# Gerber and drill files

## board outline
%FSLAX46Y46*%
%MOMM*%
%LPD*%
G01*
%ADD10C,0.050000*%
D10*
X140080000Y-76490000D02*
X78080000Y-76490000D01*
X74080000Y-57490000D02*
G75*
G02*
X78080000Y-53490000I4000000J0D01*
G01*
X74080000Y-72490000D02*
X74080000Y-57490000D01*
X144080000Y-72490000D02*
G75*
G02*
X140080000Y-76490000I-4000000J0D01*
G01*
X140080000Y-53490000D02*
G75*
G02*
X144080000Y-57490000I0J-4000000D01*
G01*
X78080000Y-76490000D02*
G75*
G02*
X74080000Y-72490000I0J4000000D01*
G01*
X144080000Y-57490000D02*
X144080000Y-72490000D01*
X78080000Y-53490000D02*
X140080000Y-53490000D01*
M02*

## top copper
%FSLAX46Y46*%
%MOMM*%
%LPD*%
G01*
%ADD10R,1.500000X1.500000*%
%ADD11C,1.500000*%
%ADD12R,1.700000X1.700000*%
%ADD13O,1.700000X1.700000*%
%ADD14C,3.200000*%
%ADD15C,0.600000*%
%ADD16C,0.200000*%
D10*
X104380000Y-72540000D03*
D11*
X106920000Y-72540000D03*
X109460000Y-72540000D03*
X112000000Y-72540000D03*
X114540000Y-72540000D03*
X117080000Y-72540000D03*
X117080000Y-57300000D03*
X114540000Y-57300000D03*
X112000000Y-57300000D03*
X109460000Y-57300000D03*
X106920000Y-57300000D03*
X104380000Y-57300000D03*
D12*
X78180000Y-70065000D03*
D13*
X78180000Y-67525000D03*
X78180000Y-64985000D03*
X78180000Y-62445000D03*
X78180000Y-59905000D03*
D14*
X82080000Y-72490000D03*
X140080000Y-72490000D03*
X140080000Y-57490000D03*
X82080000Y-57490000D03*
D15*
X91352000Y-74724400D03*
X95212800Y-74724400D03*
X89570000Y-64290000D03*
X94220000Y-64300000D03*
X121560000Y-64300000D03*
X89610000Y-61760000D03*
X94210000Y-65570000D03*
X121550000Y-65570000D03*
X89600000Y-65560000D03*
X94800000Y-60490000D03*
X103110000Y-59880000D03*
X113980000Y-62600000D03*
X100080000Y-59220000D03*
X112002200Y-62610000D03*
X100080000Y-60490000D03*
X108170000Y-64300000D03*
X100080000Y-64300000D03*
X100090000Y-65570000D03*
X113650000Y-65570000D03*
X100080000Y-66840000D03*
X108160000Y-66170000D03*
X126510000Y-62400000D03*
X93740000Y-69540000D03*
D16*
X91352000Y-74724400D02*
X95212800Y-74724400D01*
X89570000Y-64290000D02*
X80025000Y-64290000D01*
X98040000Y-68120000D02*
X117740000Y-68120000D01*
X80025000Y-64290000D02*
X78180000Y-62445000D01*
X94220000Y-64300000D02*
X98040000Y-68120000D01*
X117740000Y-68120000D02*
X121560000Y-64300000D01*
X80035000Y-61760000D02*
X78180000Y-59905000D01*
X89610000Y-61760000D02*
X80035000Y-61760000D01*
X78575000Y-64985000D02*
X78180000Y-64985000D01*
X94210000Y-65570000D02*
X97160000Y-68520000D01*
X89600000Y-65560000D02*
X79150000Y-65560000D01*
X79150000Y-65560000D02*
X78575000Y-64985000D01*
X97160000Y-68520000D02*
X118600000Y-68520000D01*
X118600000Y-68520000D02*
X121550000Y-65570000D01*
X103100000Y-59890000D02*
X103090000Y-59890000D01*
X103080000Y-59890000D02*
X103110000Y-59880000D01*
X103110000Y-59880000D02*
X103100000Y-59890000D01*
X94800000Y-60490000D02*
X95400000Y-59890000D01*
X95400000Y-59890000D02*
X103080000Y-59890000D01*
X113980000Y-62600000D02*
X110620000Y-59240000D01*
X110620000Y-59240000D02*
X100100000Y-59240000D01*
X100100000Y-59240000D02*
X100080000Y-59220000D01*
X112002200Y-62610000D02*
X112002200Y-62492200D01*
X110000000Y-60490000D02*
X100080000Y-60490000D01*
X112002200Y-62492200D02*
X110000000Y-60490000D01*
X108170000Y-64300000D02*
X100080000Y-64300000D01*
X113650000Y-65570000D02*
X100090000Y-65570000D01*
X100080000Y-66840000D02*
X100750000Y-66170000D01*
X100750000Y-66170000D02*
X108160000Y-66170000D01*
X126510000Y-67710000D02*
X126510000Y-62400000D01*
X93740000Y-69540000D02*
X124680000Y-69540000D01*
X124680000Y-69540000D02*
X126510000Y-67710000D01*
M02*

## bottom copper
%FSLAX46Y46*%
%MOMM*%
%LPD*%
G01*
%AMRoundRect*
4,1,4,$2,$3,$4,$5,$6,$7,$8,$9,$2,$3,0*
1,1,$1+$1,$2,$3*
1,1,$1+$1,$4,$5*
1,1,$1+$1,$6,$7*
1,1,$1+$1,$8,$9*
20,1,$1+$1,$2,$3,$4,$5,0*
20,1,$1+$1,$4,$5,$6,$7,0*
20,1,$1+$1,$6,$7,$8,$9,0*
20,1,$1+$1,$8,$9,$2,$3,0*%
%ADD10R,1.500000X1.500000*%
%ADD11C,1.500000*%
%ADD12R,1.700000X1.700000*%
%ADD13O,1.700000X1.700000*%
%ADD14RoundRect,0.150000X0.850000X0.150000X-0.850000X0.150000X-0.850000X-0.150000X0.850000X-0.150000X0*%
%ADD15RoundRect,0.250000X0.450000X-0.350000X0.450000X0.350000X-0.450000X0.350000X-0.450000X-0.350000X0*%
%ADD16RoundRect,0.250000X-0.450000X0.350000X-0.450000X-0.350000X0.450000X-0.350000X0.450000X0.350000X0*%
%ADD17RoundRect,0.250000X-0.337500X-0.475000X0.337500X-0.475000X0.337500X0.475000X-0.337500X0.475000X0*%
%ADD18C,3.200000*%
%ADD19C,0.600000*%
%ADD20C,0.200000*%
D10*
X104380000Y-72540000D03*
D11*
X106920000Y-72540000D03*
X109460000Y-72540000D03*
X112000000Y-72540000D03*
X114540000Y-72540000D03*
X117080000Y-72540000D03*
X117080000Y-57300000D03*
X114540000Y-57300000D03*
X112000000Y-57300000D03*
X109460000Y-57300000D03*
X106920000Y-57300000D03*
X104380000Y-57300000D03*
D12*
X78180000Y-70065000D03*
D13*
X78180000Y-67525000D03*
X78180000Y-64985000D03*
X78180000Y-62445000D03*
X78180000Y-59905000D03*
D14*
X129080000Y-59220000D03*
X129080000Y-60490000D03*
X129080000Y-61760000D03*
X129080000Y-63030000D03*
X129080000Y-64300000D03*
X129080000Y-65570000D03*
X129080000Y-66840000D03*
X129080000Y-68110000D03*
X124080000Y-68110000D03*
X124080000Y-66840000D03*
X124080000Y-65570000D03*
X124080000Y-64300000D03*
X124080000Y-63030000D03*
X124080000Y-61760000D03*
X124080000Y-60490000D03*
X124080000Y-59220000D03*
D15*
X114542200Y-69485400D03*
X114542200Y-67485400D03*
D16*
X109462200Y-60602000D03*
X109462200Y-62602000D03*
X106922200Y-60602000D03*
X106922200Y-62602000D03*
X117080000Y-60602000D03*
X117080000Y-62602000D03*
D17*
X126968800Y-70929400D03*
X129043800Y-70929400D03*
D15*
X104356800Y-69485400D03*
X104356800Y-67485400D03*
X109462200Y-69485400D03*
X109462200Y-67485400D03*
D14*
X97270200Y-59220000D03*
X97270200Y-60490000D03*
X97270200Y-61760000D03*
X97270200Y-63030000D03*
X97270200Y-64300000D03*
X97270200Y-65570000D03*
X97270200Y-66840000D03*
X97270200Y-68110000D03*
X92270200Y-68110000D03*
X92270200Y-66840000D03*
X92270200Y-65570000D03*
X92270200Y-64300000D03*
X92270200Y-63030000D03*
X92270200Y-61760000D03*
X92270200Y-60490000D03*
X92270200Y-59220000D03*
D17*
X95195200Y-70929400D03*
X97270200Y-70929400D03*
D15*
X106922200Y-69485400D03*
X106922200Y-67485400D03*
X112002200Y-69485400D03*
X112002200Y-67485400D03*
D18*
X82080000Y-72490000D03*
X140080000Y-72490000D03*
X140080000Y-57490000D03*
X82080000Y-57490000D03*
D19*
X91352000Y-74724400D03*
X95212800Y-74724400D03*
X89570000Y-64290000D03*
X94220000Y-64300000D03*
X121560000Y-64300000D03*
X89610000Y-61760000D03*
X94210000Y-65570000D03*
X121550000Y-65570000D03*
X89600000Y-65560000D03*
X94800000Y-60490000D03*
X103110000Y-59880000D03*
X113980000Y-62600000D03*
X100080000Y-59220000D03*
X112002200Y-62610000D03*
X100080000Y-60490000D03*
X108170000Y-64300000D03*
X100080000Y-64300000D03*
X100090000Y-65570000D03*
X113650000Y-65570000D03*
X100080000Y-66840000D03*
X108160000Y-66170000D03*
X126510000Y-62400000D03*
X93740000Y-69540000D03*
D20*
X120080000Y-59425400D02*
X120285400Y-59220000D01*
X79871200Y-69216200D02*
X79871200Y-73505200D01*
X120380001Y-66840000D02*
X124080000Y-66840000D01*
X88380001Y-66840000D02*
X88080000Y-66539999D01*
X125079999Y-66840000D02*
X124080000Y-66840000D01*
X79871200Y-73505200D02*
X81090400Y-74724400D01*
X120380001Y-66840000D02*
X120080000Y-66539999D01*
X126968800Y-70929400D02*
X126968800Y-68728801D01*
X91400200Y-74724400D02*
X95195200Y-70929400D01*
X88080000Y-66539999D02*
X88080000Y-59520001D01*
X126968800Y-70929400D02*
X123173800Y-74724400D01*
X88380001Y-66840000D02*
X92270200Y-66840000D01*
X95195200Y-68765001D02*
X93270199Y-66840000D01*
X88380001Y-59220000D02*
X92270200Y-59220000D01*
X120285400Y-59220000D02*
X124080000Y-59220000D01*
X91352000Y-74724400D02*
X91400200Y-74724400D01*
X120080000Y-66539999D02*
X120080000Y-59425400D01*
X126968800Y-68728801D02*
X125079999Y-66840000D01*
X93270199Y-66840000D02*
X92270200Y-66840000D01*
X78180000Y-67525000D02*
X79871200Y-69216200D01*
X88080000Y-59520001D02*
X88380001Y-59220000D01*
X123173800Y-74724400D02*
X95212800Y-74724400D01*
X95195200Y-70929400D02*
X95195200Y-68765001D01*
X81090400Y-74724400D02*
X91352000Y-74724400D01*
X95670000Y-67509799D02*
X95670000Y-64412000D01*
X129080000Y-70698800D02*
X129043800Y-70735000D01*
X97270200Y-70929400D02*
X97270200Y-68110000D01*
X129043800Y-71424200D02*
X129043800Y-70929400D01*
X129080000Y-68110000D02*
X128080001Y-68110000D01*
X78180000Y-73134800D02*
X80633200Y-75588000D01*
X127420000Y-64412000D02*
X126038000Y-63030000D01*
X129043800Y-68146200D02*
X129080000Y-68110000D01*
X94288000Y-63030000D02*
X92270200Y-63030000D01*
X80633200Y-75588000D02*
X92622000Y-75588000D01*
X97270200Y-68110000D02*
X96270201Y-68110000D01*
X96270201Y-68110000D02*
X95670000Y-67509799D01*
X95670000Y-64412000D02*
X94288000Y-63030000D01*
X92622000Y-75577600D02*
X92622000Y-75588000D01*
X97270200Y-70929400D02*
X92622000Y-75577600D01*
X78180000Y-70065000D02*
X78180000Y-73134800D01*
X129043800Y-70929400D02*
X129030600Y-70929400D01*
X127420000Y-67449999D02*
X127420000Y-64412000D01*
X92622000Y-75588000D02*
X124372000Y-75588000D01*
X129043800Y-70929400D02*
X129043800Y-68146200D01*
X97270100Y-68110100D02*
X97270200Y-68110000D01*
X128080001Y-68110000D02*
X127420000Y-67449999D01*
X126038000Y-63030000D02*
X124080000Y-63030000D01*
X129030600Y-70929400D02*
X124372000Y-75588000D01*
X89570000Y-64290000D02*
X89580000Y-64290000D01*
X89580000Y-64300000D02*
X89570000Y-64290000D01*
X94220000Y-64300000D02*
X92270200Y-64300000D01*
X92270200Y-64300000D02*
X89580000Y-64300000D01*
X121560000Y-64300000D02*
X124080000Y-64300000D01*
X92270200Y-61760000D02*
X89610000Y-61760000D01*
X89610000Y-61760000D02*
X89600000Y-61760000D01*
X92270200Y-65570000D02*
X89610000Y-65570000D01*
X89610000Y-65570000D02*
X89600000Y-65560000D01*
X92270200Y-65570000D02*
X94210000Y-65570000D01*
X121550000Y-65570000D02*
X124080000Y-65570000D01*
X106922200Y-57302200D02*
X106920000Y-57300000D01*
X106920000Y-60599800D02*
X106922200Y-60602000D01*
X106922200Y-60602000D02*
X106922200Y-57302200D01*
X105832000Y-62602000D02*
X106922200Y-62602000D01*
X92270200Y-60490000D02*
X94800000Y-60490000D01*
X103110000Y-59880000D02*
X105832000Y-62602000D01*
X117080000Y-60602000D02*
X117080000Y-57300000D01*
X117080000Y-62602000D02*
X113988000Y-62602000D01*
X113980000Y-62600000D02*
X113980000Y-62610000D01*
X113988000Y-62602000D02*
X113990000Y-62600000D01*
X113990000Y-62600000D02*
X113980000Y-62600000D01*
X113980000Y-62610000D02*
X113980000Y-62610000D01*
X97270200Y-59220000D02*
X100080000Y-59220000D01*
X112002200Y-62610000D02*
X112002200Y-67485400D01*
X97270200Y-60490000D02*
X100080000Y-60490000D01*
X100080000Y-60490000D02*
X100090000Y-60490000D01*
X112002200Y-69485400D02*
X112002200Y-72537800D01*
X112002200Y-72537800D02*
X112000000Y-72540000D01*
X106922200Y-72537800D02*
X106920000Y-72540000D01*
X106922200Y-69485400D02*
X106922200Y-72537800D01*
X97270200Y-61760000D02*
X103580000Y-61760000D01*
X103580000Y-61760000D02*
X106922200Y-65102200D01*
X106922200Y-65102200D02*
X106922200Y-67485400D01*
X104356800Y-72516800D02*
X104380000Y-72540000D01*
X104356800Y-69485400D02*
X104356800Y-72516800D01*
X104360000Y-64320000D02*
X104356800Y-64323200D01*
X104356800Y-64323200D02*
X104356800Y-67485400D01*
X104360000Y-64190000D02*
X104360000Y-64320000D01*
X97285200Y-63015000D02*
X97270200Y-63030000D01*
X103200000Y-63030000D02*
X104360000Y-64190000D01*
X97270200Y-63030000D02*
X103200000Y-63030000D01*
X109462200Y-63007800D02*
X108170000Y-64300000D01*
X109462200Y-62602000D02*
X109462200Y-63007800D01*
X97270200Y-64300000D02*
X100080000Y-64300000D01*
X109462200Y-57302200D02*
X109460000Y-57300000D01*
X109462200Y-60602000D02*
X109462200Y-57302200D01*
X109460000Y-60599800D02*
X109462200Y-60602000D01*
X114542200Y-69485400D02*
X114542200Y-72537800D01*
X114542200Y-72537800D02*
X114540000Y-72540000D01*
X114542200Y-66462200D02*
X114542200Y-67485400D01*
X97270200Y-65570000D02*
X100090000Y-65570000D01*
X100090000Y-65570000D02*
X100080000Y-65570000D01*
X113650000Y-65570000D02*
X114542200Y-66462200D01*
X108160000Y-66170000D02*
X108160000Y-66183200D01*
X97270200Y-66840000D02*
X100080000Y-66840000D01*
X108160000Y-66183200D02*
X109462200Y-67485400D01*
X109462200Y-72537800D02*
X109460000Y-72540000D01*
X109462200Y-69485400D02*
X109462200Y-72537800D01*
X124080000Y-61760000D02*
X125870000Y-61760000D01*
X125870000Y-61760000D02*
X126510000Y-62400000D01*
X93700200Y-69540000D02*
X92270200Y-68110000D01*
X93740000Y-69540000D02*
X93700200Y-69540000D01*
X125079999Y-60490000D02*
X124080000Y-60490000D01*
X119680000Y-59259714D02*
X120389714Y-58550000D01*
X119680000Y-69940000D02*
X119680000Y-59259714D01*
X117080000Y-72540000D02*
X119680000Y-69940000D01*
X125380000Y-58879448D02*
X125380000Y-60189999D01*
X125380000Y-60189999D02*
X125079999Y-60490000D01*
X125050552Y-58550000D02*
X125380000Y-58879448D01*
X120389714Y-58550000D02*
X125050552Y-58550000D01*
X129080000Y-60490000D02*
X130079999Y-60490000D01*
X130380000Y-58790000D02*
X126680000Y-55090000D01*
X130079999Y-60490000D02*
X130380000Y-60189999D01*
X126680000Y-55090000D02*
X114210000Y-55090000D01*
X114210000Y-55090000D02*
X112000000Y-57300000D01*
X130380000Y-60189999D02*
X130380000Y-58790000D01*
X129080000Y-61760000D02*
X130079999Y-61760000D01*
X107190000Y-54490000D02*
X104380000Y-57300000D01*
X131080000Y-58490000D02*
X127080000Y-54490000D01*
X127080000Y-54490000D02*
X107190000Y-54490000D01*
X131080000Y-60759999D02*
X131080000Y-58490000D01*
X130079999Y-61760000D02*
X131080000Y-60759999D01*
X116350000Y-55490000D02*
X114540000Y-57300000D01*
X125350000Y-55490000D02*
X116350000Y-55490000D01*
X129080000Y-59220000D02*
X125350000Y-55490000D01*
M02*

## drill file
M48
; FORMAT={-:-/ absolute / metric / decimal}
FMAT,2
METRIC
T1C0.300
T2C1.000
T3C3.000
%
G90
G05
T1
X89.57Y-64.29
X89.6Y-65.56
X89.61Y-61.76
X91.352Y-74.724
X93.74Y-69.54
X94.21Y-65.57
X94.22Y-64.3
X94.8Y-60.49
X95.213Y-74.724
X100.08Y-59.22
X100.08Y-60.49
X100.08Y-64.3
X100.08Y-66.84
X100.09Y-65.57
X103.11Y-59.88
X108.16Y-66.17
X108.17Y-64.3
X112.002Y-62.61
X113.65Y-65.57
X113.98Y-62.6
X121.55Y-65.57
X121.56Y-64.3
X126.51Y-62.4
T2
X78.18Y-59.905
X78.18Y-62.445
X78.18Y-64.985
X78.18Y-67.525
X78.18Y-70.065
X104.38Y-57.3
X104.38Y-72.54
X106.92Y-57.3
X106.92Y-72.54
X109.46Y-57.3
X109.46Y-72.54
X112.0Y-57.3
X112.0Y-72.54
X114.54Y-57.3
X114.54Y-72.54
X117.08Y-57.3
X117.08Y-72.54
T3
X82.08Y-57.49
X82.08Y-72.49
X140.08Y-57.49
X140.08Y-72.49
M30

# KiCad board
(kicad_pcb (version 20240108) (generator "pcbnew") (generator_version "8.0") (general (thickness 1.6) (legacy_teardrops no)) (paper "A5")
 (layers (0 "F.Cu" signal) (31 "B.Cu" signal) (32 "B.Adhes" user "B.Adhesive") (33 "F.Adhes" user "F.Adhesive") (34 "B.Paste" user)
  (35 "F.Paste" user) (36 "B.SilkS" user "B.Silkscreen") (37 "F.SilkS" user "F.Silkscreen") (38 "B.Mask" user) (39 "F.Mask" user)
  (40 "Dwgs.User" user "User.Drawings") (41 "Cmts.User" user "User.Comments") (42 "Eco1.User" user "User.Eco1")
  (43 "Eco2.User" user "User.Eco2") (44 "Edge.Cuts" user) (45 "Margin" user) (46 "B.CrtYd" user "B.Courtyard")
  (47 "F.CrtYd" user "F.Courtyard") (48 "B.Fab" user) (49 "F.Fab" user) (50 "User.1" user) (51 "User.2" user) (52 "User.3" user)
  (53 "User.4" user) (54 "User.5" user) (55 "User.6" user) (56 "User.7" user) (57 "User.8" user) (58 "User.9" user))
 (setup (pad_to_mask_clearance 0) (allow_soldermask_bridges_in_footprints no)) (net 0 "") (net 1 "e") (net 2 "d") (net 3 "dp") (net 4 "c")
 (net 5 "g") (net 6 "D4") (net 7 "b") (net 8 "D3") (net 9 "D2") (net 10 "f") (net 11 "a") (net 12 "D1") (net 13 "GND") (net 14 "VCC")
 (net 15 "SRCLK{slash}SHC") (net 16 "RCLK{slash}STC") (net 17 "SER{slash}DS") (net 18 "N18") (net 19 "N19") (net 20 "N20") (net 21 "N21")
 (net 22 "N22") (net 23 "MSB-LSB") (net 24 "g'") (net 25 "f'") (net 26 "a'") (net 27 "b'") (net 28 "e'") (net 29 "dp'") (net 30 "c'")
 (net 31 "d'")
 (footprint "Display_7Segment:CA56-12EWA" (layer "F.Cu") (at 104.38 72.54 90)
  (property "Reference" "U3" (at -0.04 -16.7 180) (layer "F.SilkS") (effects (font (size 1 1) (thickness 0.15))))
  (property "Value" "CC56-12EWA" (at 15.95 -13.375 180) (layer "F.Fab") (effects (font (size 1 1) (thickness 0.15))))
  (pad "1" thru_hole rect (at 0 0 90) (size 1.5 1.5) (drill 1) (layers "*.Cu" "*.Mask") (remove_unused_layers no) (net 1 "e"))
  (pad "2" thru_hole circle (at 0 2.54 90) (size 1.5 1.5) (drill 1) (layers "*.Cu" "*.Mask") (remove_unused_layers no) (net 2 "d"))
  (pad "3" thru_hole circle (at 0 5.08 90) (size 1.5 1.5) (drill 1) (layers "*.Cu" "*.Mask") (remove_unused_layers no) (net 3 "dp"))
  (pad "4" thru_hole circle (at 0 7.62 90) (size 1.5 1.5) (drill 1) (layers "*.Cu" "*.Mask") (remove_unused_layers no) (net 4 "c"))
  (pad "5" thru_hole circle (at 0 10.16 90) (size 1.5 1.5) (drill 1) (layers "*.Cu" "*.Mask") (remove_unused_layers no) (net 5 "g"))
  (pad "6" thru_hole circle (at 0 12.7 90) (size 1.5 1.5) (drill 1) (layers "*.Cu" "*.Mask") (remove_unused_layers no) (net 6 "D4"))
  (pad "7" thru_hole circle (at 15.24 12.7 90) (size 1.5 1.5) (drill 1) (layers "*.Cu" "*.Mask") (remove_unused_layers no) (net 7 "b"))
  (pad "8" thru_hole circle (at 15.24 10.16 90) (size 1.5 1.5) (drill 1) (layers "*.Cu" "*.Mask") (remove_unused_layers no) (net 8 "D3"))
  (pad "9" thru_hole circle (at 15.24 7.62 90) (size 1.5 1.5) (drill 1) (layers "*.Cu" "*.Mask") (remove_unused_layers no) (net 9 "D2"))
  (pad "10" thru_hole circle (at 15.24 5.08 90) (size 1.5 1.5) (drill 1) (layers "*.Cu" "*.Mask") (remove_unused_layers no) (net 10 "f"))
  (pad "11" thru_hole circle (at 15.24 2.54 90) (size 1.5 1.5) (drill 1) (layers "*.Cu" "*.Mask") (remove_unused_layers no) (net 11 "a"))
  (pad "12" thru_hole circle (at 15.24 0 90) (size 1.5 1.5) (drill 1) (layers "*.Cu" "*.Mask") (remove_unused_layers no) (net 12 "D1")))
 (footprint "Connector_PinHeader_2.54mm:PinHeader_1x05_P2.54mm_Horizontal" (layer "F.Cu") (at 78.18 70.065 180)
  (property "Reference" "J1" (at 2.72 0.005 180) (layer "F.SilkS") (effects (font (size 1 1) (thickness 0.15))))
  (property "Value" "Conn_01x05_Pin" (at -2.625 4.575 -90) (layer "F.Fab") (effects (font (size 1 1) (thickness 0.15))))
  (pad "1" thru_hole rect (at 0 0 180) (size 1.7 1.7) (drill 1) (layers "*.Cu" "*.Mask") (remove_unused_layers no) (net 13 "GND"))
  (pad "2" thru_hole oval (at 0 2.54 180) (size 1.7 1.7) (drill 1) (layers "*.Cu" "*.Mask") (remove_unused_layers no) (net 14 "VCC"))
  (pad "3" thru_hole oval (at 0 5.08 180) (size 1.7 1.7) (drill 1) (layers "*.Cu" "*.Mask") (remove_unused_layers no)
   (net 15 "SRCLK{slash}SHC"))
  (pad "4" thru_hole oval (at 0 7.62 180) (size 1.7 1.7) (drill 1) (layers "*.Cu" "*.Mask") (remove_unused_layers no)
   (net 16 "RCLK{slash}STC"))
  (pad "5" thru_hole oval (at 0 10.16 180) (size 1.7 1.7) (drill 1) (layers "*.Cu" "*.Mask") (remove_unused_layers no)
   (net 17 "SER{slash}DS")))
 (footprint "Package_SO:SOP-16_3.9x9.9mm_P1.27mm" (layer "B.Cu") (at 126.58 63.665 180)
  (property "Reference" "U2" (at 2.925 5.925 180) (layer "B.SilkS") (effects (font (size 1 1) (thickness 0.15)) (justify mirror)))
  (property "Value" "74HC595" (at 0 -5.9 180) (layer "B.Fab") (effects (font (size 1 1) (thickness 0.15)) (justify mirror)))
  (pad "1" smd roundrect (at -2.5 4.445 180) (size 2 0.6) (layers "B.Cu" "B.Paste" "B.Mask") (roundrect_rratio 0.25) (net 8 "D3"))
  (pad "2" smd roundrect (at -2.5 3.175 180) (size 2 0.6) (layers "B.Cu" "B.Paste" "B.Mask") (roundrect_rratio 0.25) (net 9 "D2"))
  (pad "3" smd roundrect (at -2.5 1.905 180) (size 2 0.6) (layers "B.Cu" "B.Paste" "B.Mask") (roundrect_rratio 0.25) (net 12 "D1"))
  (pad "4" smd roundrect (at -2.5 0.635 180) (size 2 0.6) (layers "B.Cu" "B.Paste" "B.Mask") (roundrect_rratio 0.25) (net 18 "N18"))
  (pad "5" smd roundrect (at -2.5 -0.635 180) (size 2 0.6) (layers "B.Cu" "B.Paste" "B.Mask") (roundrect_rratio 0.25) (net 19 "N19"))
  (pad "6" smd roundrect (at -2.5 -1.905 180) (size 2 0.6) (layers "B.Cu" "B.Paste" "B.Mask") (roundrect_rratio 0.25) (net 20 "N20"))
  (pad "7" smd roundrect (at -2.5 -3.175 180) (size 2 0.6) (layers "B.Cu" "B.Paste" "B.Mask") (roundrect_rratio 0.25) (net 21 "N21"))
  (pad "8" smd roundrect (at -2.5 -4.445 180) (size 2 0.6) (layers "B.Cu" "B.Paste" "B.Mask") (roundrect_rratio 0.25) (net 13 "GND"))
  (pad "9" smd roundrect (at 2.5 -4.445 180) (size 2 0.6) (layers "B.Cu" "B.Paste" "B.Mask") (roundrect_rratio 0.25) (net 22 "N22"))
  (pad "10" smd roundrect (at 2.5 -3.175 180) (size 2 0.6) (layers "B.Cu" "B.Paste" "B.Mask") (roundrect_rratio 0.25) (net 14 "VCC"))
  (pad "11" smd roundrect (at 2.5 -1.905 180) (size 2 0.6) (layers "B.Cu" "B.Paste" "B.Mask") (roundrect_rratio 0.25)
   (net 15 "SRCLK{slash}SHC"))
  (pad "12" smd roundrect (at 2.5 -0.635 180) (size 2 0.6) (layers "B.Cu" "B.Paste" "B.Mask") (roundrect_rratio 0.25)
   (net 16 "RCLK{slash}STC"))
  (pad "13" smd roundrect (at 2.5 0.635 180) (size 2 0.6) (layers "B.Cu" "B.Paste" "B.Mask") (roundrect_rratio 0.25) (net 13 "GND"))
  (pad "14" smd roundrect (at 2.5 1.905 180) (size 2 0.6) (layers "B.Cu" "B.Paste" "B.Mask") (roundrect_rratio 0.25) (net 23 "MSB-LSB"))
  (pad "15" smd roundrect (at 2.5 3.175 180) (size 2 0.6) (layers "B.Cu" "B.Paste" "B.Mask") (roundrect_rratio 0.25) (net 6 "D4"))
  (pad "16" smd roundrect (at 2.5 4.445 180) (size 2 0.6) (layers "B.Cu" "B.Paste" "B.Mask") (roundrect_rratio 0.25) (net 14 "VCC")))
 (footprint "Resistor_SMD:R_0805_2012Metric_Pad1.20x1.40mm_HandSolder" (layer "B.Cu") (at 114.5422 68.4854 90)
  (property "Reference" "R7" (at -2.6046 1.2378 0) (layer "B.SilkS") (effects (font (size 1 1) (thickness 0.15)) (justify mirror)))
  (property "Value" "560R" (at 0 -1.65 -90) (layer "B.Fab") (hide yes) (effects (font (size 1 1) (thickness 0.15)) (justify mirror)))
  (pad "1" smd roundrect (at -1 0 90) (size 1.2 1.4) (layers "B.Cu" "B.Paste" "B.Mask") (roundrect_rratio 0.208333) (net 5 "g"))
  (pad "2" smd roundrect (at 1 0 90) (size 1.2 1.4) (layers "B.Cu" "B.Paste" "B.Mask") (roundrect_rratio 0.208333) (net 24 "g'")))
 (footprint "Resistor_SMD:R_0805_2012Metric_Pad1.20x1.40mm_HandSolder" (layer "B.Cu") (at 109.4622 61.602 -90)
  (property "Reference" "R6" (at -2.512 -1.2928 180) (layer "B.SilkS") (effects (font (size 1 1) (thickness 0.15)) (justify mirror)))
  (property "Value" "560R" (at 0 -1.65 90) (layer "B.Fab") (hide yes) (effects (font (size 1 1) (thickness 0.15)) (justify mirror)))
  (pad "1" smd roundrect (at -1 0 270) (size 1.2 1.4) (layers "B.Cu" "B.Paste" "B.Mask") (roundrect_rratio 0.208333) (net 10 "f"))
  (pad "2" smd roundrect (at 1 0 270) (size 1.2 1.4) (layers "B.Cu" "B.Paste" "B.Mask") (roundrect_rratio 0.208333) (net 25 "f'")))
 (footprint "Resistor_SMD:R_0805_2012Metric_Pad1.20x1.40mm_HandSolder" (layer "B.Cu") (at 106.9222 61.602 -90)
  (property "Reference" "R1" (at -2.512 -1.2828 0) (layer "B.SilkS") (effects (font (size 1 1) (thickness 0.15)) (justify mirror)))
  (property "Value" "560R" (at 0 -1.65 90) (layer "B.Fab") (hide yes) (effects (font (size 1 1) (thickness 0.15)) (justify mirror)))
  (pad "1" smd roundrect (at -1 0 270) (size 1.2 1.4) (layers "B.Cu" "B.Paste" "B.Mask") (roundrect_rratio 0.208333) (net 11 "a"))
  (pad "2" smd roundrect (at 1 0 270) (size 1.2 1.4) (layers "B.Cu" "B.Paste" "B.Mask") (roundrect_rratio 0.208333) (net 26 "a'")))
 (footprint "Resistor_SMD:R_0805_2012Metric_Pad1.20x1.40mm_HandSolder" (layer "B.Cu") (at 117.08 61.602 -90)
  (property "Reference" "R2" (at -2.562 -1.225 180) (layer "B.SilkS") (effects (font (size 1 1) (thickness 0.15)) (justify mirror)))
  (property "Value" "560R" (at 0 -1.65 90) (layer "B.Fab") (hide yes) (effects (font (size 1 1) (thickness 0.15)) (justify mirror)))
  (pad "1" smd roundrect (at -1 0 270) (size 1.2 1.4) (layers "B.Cu" "B.Paste" "B.Mask") (roundrect_rratio 0.208333) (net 7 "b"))
  (pad "2" smd roundrect (at 1 0 270) (size 1.2 1.4) (layers "B.Cu" "B.Paste" "B.Mask") (roundrect_rratio 0.208333) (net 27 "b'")))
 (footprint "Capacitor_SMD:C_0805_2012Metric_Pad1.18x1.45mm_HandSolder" (layer "B.Cu") (at 128.0063 70.9294)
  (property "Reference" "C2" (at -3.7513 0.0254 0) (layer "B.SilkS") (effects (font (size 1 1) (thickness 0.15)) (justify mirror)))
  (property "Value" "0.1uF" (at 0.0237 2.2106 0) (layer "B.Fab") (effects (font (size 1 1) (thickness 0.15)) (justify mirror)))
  (pad "1" smd roundrect (at -1.0375 0) (size 1.175 1.45) (layers "B.Cu" "B.Paste" "B.Mask") (roundrect_rratio 0.212766) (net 14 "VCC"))
  (pad "2" smd roundrect (at 1.0375 0) (size 1.175 1.45) (layers "B.Cu" "B.Paste" "B.Mask") (roundrect_rratio 0.212766) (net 13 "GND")))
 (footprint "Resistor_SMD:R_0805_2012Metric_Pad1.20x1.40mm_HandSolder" (layer "B.Cu") (at 104.3568 68.4854 90)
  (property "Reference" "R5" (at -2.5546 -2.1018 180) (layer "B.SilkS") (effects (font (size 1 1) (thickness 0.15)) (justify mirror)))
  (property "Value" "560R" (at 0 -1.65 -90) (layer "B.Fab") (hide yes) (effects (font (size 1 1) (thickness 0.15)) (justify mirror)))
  (pad "1" smd roundrect (at -1 0 90) (size 1.2 1.4) (layers "B.Cu" "B.Paste" "B.Mask") (roundrect_rratio 0.208333) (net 1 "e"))
  (pad "2" smd roundrect (at 1 0 90) (size 1.2 1.4) (layers "B.Cu" "B.Paste" "B.Mask") (roundrect_rratio 0.208333) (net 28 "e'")))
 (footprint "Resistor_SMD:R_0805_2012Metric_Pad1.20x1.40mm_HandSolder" (layer "B.Cu") (at 109.4622 68.4854 90)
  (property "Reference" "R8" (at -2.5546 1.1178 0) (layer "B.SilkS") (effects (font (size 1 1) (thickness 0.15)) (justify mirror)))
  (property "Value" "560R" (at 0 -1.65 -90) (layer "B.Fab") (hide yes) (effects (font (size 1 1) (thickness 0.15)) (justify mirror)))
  (pad "1" smd roundrect (at -1 0 90) (size 1.2 1.4) (layers "B.Cu" "B.Paste" "B.Mask") (roundrect_rratio 0.208333) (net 3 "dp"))
  (pad "2" smd roundrect (at 1 0 90) (size 1.2 1.4) (layers "B.Cu" "B.Paste" "B.Mask") (roundrect_rratio 0.208333) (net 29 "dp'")))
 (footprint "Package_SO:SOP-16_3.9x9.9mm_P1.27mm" (layer "B.Cu") (at 94.7702 63.665 180)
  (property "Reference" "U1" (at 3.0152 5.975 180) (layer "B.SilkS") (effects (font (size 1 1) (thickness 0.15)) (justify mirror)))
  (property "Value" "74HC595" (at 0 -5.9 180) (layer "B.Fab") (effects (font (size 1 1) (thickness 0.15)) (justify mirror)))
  (pad "1" smd roundrect (at -2.5 4.445 180) (size 2 0.6) (layers "B.Cu" "B.Paste" "B.Mask") (roundrect_rratio 0.25) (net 27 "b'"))
  (pad "2" smd roundrect (at -2.5 3.175 180) (size 2 0.6) (layers "B.Cu" "B.Paste" "B.Mask") (roundrect_rratio 0.25) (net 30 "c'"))
  (pad "3" smd roundrect (at -2.5 1.905 180) (size 2 0.6) (layers "B.Cu" "B.Paste" "B.Mask") (roundrect_rratio 0.25) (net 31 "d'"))
  (pad "4" smd roundrect (at -2.5 0.635 180) (size 2 0.6) (layers "B.Cu" "B.Paste" "B.Mask") (roundrect_rratio 0.25) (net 28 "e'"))
  (pad "5" smd roundrect (at -2.5 -0.635 180) (size 2 0.6) (layers "B.Cu" "B.Paste" "B.Mask") (roundrect_rratio 0.25) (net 25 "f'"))
  (pad "6" smd roundrect (at -2.5 -1.905 180) (size 2 0.6) (layers "B.Cu" "B.Paste" "B.Mask") (roundrect_rratio 0.25) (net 24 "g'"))
  (pad "7" smd roundrect (at -2.5 -3.175 180) (size 2 0.6) (layers "B.Cu" "B.Paste" "B.Mask") (roundrect_rratio 0.25) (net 29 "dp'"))
  (pad "8" smd roundrect (at -2.5 -4.445 180) (size 2 0.6) (layers "B.Cu" "B.Paste" "B.Mask") (roundrect_rratio 0.25) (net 13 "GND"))
  (pad "9" smd roundrect (at 2.5 -4.445 180) (size 2 0.6) (layers "B.Cu" "B.Paste" "B.Mask") (roundrect_rratio 0.25) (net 23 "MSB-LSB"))
  (pad "10" smd roundrect (at 2.5 -3.175 180) (size 2 0.6) (layers "B.Cu" "B.Paste" "B.Mask") (roundrect_rratio 0.25) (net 14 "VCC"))
  (pad "11" smd roundrect (at 2.5 -1.905 180) (size 2 0.6) (layers "B.Cu" "B.Paste" "B.Mask") (roundrect_rratio 0.25)
   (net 15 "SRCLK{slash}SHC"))
  (pad "12" smd roundrect (at 2.5 -0.635 180) (size 2 0.6) (layers "B.Cu" "B.Paste" "B.Mask") (roundrect_rratio 0.25)
   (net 16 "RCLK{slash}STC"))
  (pad "13" smd roundrect (at 2.5 0.635 180) (size 2 0.6) (layers "B.Cu" "B.Paste" "B.Mask") (roundrect_rratio 0.25) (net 13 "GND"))
  (pad "14" smd roundrect (at 2.5 1.905 180) (size 2 0.6) (layers "B.Cu" "B.Paste" "B.Mask") (roundrect_rratio 0.25) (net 17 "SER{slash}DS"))
  (pad "15" smd roundrect (at 2.5 3.175 180) (size 2 0.6) (layers "B.Cu" "B.Paste" "B.Mask") (roundrect_rratio 0.25) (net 26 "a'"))
  (pad "16" smd roundrect (at 2.5 4.445 180) (size 2 0.6) (layers "B.Cu" "B.Paste" "B.Mask") (roundrect_rratio 0.25) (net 14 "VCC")))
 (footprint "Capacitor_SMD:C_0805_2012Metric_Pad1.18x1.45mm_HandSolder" (layer "B.Cu") (at 96.2327 70.9294)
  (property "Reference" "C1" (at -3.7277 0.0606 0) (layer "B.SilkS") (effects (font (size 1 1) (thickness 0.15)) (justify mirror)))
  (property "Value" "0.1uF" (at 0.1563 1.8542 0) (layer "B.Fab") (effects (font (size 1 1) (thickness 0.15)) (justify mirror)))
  (pad "1" smd roundrect (at -1.0375 0) (size 1.175 1.45) (layers "B.Cu" "B.Paste" "B.Mask") (roundrect_rratio 0.212766) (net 14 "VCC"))
  (pad "2" smd roundrect (at 1.0375 0) (size 1.175 1.45) (layers "B.Cu" "B.Paste" "B.Mask") (roundrect_rratio 0.212766) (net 13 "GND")))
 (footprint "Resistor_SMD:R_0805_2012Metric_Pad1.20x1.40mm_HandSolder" (layer "B.Cu") (at 106.9222 68.4854 90)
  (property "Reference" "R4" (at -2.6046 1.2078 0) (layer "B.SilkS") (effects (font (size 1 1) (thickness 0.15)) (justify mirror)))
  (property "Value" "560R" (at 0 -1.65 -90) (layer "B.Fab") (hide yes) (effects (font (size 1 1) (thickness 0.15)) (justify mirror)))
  (pad "1" smd roundrect (at -1 0 90) (size 1.2 1.4) (layers "B.Cu" "B.Paste" "B.Mask") (roundrect_rratio 0.208333) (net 2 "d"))
  (pad "2" smd roundrect (at 1 0 90) (size 1.2 1.4) (layers "B.Cu" "B.Paste" "B.Mask") (roundrect_rratio 0.208333) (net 31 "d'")))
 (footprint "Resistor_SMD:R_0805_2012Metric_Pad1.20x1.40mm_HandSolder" (layer "B.Cu") (at 112.0022 68.4854 90)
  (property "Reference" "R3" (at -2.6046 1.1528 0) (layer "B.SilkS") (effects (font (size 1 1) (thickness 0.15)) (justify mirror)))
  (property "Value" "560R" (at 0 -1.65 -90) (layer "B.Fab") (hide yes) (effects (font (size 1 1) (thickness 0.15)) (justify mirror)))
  (pad "1" smd roundrect (at -1 0 90) (size 1.2 1.4) (layers "B.Cu" "B.Paste" "B.Mask") (roundrect_rratio 0.208333) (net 4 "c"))
  (pad "2" smd roundrect (at 1 0 90) (size 1.2 1.4) (layers "B.Cu" "B.Paste" "B.Mask") (roundrect_rratio 0.208333) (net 30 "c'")))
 (gr_line (start 140.08 76.49) (end 78.08 76.49) (stroke (width 0.05) (type default)) (layer "Edge.Cuts"))
 (gr_arc (start 74.08 57.49) (mid 75.251573 54.661573) (end 78.08 53.49) (stroke (width 0.05) (type default)) (layer "Edge.Cuts"))
 (gr_line (start 74.08 72.49) (end 74.08 57.49) (stroke (width 0.05) (type default)) (layer "Edge.Cuts"))
 (gr_arc (start 144.08 72.49) (mid 142.908427 75.318427) (end 140.08 76.49) (stroke (width 0.05) (type default)) (layer "Edge.Cuts"))
 (gr_arc (start 140.08 53.49) (mid 142.908427 54.661573) (end 144.08 57.49) (stroke (width 0.05) (type default)) (layer "Edge.Cuts"))
 (gr_arc (start 78.08 76.49) (mid 75.251573 75.318427) (end 74.08 72.49) (stroke (width 0.05) (type default)) (layer "Edge.Cuts"))
 (gr_line (start 144.08 57.49) (end 144.08 72.49) (stroke (width 0.05) (type default)) (layer "Edge.Cuts"))
 (gr_line (start 78.08 53.49) (end 140.08 53.49) (stroke (width 0.05) (type default)) (layer "Edge.Cuts"))
 (via (at 82.08 72.49) (size 3.2) (drill 3) (layers "F.Cu" "B.Cu") (free yes) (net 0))
 (via (at 140.08 72.49) (size 3.2) (drill 3) (layers "F.Cu" "B.Cu") (free yes) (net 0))
 (via (at 140.08 57.49) (size 3.2) (drill 3) (layers "F.Cu" "B.Cu") (free yes) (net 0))
 (via (at 82.08 57.49) (size 3.2) (drill 3) (layers "F.Cu" "B.Cu") (free yes) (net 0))
 (segment (start 91.352 74.7244) (end 95.2128 74.7244) (width 0.2) (layer "F.Cu") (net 14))
 (via (at 91.352 74.7244) (size 0.6) (drill 0.3) (layers "F.Cu" "B.Cu") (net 14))
 (via (at 95.2128 74.7244) (size 0.6) (drill 0.3) (layers "F.Cu" "B.Cu") (free yes) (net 14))
 (segment (start 120.08 59.4254) (end 120.2854 59.22) (width 0.2) (layer "B.Cu") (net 14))
 (segment (start 79.8712 69.2162) (end 79.8712 73.5052) (width 0.2) (layer "B.Cu") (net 14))
 (segment (start 120.380001 66.84) (end 124.08 66.84) (width 0.2) (layer "B.Cu") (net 14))
 (segment (start 88.380001 66.84) (end 88.08 66.539999) (width 0.2) (layer "B.Cu") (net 14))
 (segment (start 125.079999 66.84) (end 124.08 66.84) (width 0.2) (layer "B.Cu") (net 14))
 (segment (start 79.8712 73.5052) (end 81.0904 74.7244) (width 0.2) (layer "B.Cu") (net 14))
 (segment (start 120.380001 66.84) (end 120.08 66.539999) (width 0.2) (layer "B.Cu") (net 14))
 (segment (start 126.9688 70.9294) (end 126.9688 68.728801) (width 0.2) (layer "B.Cu") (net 14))
 (segment (start 91.4002 74.7244) (end 95.1952 70.9294) (width 0.2) (layer "B.Cu") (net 14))
 (segment (start 88.08 66.539999) (end 88.08 59.520001) (width 0.2) (layer "B.Cu") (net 14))
 (segment (start 126.9688 70.9294) (end 123.1738 74.7244) (width 0.2) (layer "B.Cu") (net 14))
 (segment (start 88.380001 66.84) (end 92.2702 66.84) (width 0.2) (layer "B.Cu") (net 14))
 (segment (start 95.1952 68.765001) (end 93.270199 66.84) (width 0.2) (layer "B.Cu") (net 14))
 (segment (start 88.380001 59.22) (end 92.2702 59.22) (width 0.2) (layer "B.Cu") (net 14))
 (segment (start 120.2854 59.22) (end 124.08 59.22) (width 0.2) (layer "B.Cu") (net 14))
 (segment (start 91.352 74.7244) (end 91.4002 74.7244) (width 0.2) (layer "B.Cu") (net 14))
 (segment (start 120.08 66.539999) (end 120.08 59.4254) (width 0.2) (layer "B.Cu") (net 14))
 (segment (start 126.9688 68.728801) (end 125.079999 66.84) (width 0.2) (layer "B.Cu") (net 14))
 (segment (start 93.270199 66.84) (end 92.2702 66.84) (width 0.2) (layer "B.Cu") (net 14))
 (segment (start 78.18 67.525) (end 79.8712 69.2162) (width 0.2) (layer "B.Cu") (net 14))
 (segment (start 88.08 59.520001) (end 88.380001 59.22) (width 0.2) (layer "B.Cu") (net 14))
 (segment (start 123.1738 74.7244) (end 95.2128 74.7244) (width 0.2) (layer "B.Cu") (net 14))
 (segment (start 95.1952 70.9294) (end 95.1952 68.765001) (width 0.2) (layer "B.Cu") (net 14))
 (segment (start 81.0904 74.7244) (end 91.352 74.7244) (width 0.2) (layer "B.Cu") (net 14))
 (segment (start 95.67 67.509799) (end 95.67 64.412) (width 0.2) (layer "B.Cu") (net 13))
 (segment (start 129.08 70.6988) (end 129.0438 70.735) (width 0.2) (layer "B.Cu") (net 13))
 (segment (start 97.2702 70.9294) (end 97.2702 68.11) (width 0.2) (layer "B.Cu") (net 13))
 (segment (start 129.0438 71.4242) (end 129.0438 70.9294) (width 0.2) (layer "B.Cu") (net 13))
 (segment (start 129.08 68.11) (end 128.080001 68.11) (width 0.2) (layer "B.Cu") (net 13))
 (segment (start 78.18 73.1348) (end 80.6332 75.588) (width 0.2) (layer "B.Cu") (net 13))
 (segment (start 127.42 64.412) (end 126.038 63.03) (width 0.2) (layer "B.Cu") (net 13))
 (segment (start 129.0438 68.1462) (end 129.08 68.11) (width 0.2) (layer "B.Cu") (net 13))
 (segment (start 94.288 63.03) (end 92.2702 63.03) (width 0.2) (layer "B.Cu") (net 13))
 (segment (start 80.6332 75.588) (end 92.622 75.588) (width 0.2) (layer "B.Cu") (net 13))
 (segment (start 97.2702 68.11) (end 96.270201 68.11) (width 0.2) (layer "B.Cu") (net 13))
 (segment (start 96.270201 68.11) (end 95.67 67.509799) (width 0.2) (layer "B.Cu") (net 13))
 (segment (start 95.67 64.412) (end 94.288 63.03) (width 0.2) (layer "B.Cu") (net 13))
 (segment (start 92.622 75.5776) (end 92.622 75.588) (width 0.2) (layer "B.Cu") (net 13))
 (segment (start 97.2702 70.9294) (end 92.622 75.5776) (width 0.2) (layer "B.Cu") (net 13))
 (segment (start 78.18 70.065) (end 78.18 73.1348) (width 0.2) (layer "B.Cu") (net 13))
 (segment (start 129.0438 70.9294) (end 129.0306 70.9294) (width 0.2) (layer "B.Cu") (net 13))
 (segment (start 127.42 67.449999) (end 127.42 64.412) (width 0.2) (layer "B.Cu") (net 13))
 (segment (start 92.622 75.588) (end 124.372 75.588) (width 0.2) (layer "B.Cu") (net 13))
 (segment (start 129.0438 70.9294) (end 129.0438 68.1462) (width 0.2) (layer "B.Cu") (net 13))
 (segment (start 97.2701 68.1101) (end 97.2702 68.11) (width 0.2) (layer "B.Cu") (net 13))
 (segment (start 128.080001 68.11) (end 127.42 67.449999) (width 0.2) (layer "B.Cu") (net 13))
 (segment (start 126.038 63.03) (end 124.08 63.03) (width 0.2) (layer "B.Cu") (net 13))
 (segment (start 129.0306 70.9294) (end 124.372 75.588) (width 0.2) (layer "B.Cu") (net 13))
 (segment (start 89.57 64.29) (end 80.025 64.29) (width 0.2) (layer "F.Cu") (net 16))
 (segment (start 98.04 68.12) (end 117.74 68.12) (width 0.2) (layer "F.Cu") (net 16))
 (segment (start 80.025 64.29) (end 78.18 62.445) (width 0.2) (layer "F.Cu") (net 16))
 (segment (start 94.22 64.3) (end 98.04 68.12) (width 0.2) (layer "F.Cu") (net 16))
 (segment (start 117.74 68.12) (end 121.56 64.3) (width 0.2) (layer "F.Cu") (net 16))
 (via (at 89.57 64.29) (size 0.6) (drill 0.3) (layers "F.Cu" "B.Cu") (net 16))
 (via (at 94.22 64.3) (size 0.6) (drill 0.3) (layers "F.Cu" "B.Cu") (free yes) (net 16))
 (via (at 121.56 64.3) (size 0.6) (drill 0.3) (layers "F.Cu" "B.Cu") (free yes) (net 16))
 (segment (start 89.57 64.29) (end 89.58 64.29) (width 0.2) (layer "B.Cu") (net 16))
 (segment (start 89.58 64.3) (end 89.57 64.29) (width 0.2) (layer "B.Cu") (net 16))
 (segment (start 94.22 64.3) (end 92.2702 64.3) (width 0.2) (layer "B.Cu") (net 16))
 (segment (start 92.2702 64.3) (end 89.58 64.3) (width 0.2) (layer "B.Cu") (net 16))
 (segment (start 121.56 64.3) (end 124.08 64.3) (width 0.2) (layer "B.Cu") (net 16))
 (segment (start 80.035 61.76) (end 78.18 59.905) (width 0.2) (layer "F.Cu") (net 17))
 (segment (start 89.61 61.76) (end 80.035 61.76) (width 0.2) (layer "F.Cu") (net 17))
 (via (at 89.61 61.76) (size 0.6) (drill 0.3) (layers "F.Cu" "B.Cu") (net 17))
 (segment (start 92.2702 61.76) (end 89.61 61.76) (width 0.2) (layer "B.Cu") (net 17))
 (segment (start 89.61 61.76) (end 89.6 61.76) (width 0.2) (layer "B.Cu") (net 17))
 (segment (start 78.575 64.985) (end 78.18 64.985) (width 0.2) (layer "F.Cu") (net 15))
 (segment (start 94.21 65.57) (end 97.16 68.52) (width 0.2) (layer "F.Cu") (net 15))
 (segment (start 89.6 65.56) (end 79.15 65.56) (width 0.2) (layer "F.Cu") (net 15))
 (segment (start 79.15 65.56) (end 78.575 64.985) (width 0.2) (layer "F.Cu") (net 15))
 (segment (start 97.16 68.52) (end 118.6 68.52) (width 0.2) (layer "F.Cu") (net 15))
 (segment (start 118.6 68.52) (end 121.55 65.57) (width 0.2) (layer "F.Cu") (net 15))
 (via (at 94.21 65.57) (size 0.6) (drill 0.3) (layers "F.Cu" "B.Cu") (free yes) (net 15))
 (via (at 121.55 65.57) (size 0.6) (drill 0.3) (layers "F.Cu" "B.Cu") (free yes) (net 15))
 (via (at 89.6 65.56) (size 0.6) (drill 0.3) (layers "F.Cu" "B.Cu") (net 15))
 (segment (start 92.2702 65.57) (end 89.61 65.57) (width 0.2) (layer "B.Cu") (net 15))
 (segment (start 89.61 65.57) (end 89.6 65.56) (width 0.2) (layer "B.Cu") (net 15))
 (segment (start 92.2702 65.57) (end 94.21 65.57) (width 0.2) (layer "B.Cu") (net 15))
 (segment (start 121.55 65.57) (end 124.08 65.57) (width 0.2) (layer "B.Cu") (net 15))
 (segment (start 106.9222 57.3022) (end 106.92 57.3) (width 0.2) (layer "B.Cu") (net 11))
 (segment (start 106.92 60.5998) (end 106.9222 60.602) (width 0.2) (layer "B.Cu") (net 11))
 (segment (start 106.9222 60.602) (end 106.9222 57.3022) (width 0.2) (layer "B.Cu") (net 11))
 (segment (start 103.1 59.89) (end 103.09 59.89) (width 0.2) (layer "F.Cu") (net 26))
 (segment (start 103.08 59.89) (end 103.11 59.88) (width 0.2) (layer "F.Cu") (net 26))
 (segment (start 103.11 59.88) (end 103.1 59.89) (width 0.2) (layer "F.Cu") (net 26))
 (segment (start 94.8 60.49) (end 95.4 59.89) (width 0.2) (layer "F.Cu") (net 26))
 (segment (start 95.4 59.89) (end 103.08 59.89) (width 0.2) (layer "F.Cu") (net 26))
 (via (at 94.8 60.49) (size 0.6) (drill 0.3) (layers "F.Cu" "B.Cu") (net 26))
 (via (at 103.11 59.88) (size 0.6) (drill 0.3) (layers "F.Cu" "B.Cu") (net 26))
 (segment (start 105.832 62.602) (end 106.9222 62.602) (width 0.2) (layer "B.Cu") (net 26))
 (segment (start 92.2702 60.49) (end 94.8 60.49) (width 0.2) (layer "B.Cu") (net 26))
 (segment (start 103.11 59.88) (end 105.832 62.602) (width 0.2) (layer "B.Cu") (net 26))
 (segment (start 117.08 60.602) (end 117.08 57.3) (width 0.2) (layer "B.Cu") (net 7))
 (segment (start 113.98 62.6) (end 110.62 59.24) (width 0.2) (layer "F.Cu") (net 27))
 (segment (start 110.62 59.24) (end 100.1 59.24) (width 0.2) (layer "F.Cu") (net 27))
 (segment (start 100.1 59.24) (end 100.08 59.22) (width 0.2) (layer "F.Cu") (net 27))
 (via (at 113.98 62.6) (size 0.6) (drill 0.3) (layers "F.Cu" "B.Cu") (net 27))
 (via (at 100.08 59.22) (size 0.6) (drill 0.3) (layers "F.Cu" "B.Cu") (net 27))
 (segment (start 117.08 62.602) (end 113.988 62.602) (width 0.2) (layer "B.Cu") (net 27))
 (segment (start 113.98 62.6) (end 113.98 62.61) (width 0.2) (layer "B.Cu") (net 27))
 (segment (start 113.988 62.602) (end 113.99 62.6) (width 0.2) (layer "B.Cu") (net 27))
 (segment (start 113.99 62.6) (end 113.98 62.6) (width 0.2) (layer "B.Cu") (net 27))
 (segment (start 113.98 62.61) (end 113.98 62.61) (width 0.2) (layer "B.Cu") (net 27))
 (segment (start 97.2702 59.22) (end 100.08 59.22) (width 0.2) (layer "B.Cu") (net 27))
 (segment (start 112.0022 62.61) (end 112.0022 62.4922) (width 0.2) (layer "F.Cu") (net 30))
 (segment (start 110 60.49) (end 100.08 60.49) (width 0.2) (layer "F.Cu") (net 30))
 (segment (start 112.0022 62.4922) (end 110 60.49) (width 0.2) (layer "F.Cu") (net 30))
 (via (at 112.0022 62.61) (size 0.6) (drill 0.3) (layers "F.Cu" "B.Cu") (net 30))
 (via (at 100.08 60.49) (size 0.6) (drill 0.3) (layers "F.Cu" "B.Cu") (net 30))
 (segment (start 112.0022 62.61) (end 112.0022 67.4854) (width 0.2) (layer "B.Cu") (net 30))
 (segment (start 97.2702 60.49) (end 100.08 60.49) (width 0.2) (layer "B.Cu") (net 30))
 (segment (start 100.08 60.49) (end 100.09 60.49) (width 0.2) (layer "B.Cu") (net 30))
 (segment (start 112.0022 69.4854) (end 112.0022 72.5378) (width 0.2) (layer "B.Cu") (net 4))
 (segment (start 112.0022 72.5378) (end 112 72.54) (width 0.2) (layer "B.Cu") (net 4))
 (segment (start 106.9222 72.5378) (end 106.92 72.54) (width 0.2) (layer "B.Cu") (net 2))
 (segment (start 106.9222 69.4854) (end 106.9222 72.5378) (width 0.2) (layer "B.Cu") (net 2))
 (segment (start 97.2702 61.76) (end 103.58 61.76) (width 0.2) (layer "B.Cu") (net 31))
 (segment (start 103.58 61.76) (end 106.9222 65.1022) (width 0.2) (layer "B.Cu") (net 31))
 (segment (start 106.9222 65.1022) (end 106.9222 67.4854) (width 0.2) (layer "B.Cu") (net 31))
 (segment (start 104.3568 72.5168) (end 104.38 72.54) (width 0.2) (layer "B.Cu") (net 1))
 (segment (start 104.3568 69.4854) (end 104.3568 72.5168) (width 0.2) (layer "B.Cu") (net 1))
 (segment (start 104.36 64.32) (end 104.3568 64.3232) (width 0.2) (layer "B.Cu") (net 28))
 (segment (start 104.3568 64.3232) (end 104.3568 67.4854) (width 0.2) (layer "B.Cu") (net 28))
 (segment (start 104.36 64.19) (end 104.36 64.32) (width 0.2) (layer "B.Cu") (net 28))
 (segment (start 97.2852 63.015) (end 97.2702 63.03) (width 0.2) (layer "B.Cu") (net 28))
 (segment (start 103.2 63.03) (end 104.36 64.19) (width 0.2) (layer "B.Cu") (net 28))
 (segment (start 97.2702 63.03) (end 103.2 63.03) (width 0.2) (layer "B.Cu") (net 28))
 (segment (start 108.17 64.3) (end 100.08 64.3) (width 0.2) (layer "F.Cu") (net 25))
 (via (at 108.17 64.3) (size 0.6) (drill 0.3) (layers "F.Cu" "B.Cu") (free yes) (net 25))
 (via (at 100.08 64.3) (size 0.6) (drill 0.3) (layers "F.Cu" "B.Cu") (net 25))
 (segment (start 109.4622 63.0078) (end 108.17 64.3) (width 0.2) (layer "B.Cu") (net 25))
 (segment (start 109.4622 62.602) (end 109.4622 63.0078) (width 0.2) (layer "B.Cu") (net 25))
 (segment (start 97.2702 64.3) (end 100.08 64.3) (width 0.2) (layer "B.Cu") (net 25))
 (segment (start 109.4622 57.3022) (end 109.46 57.3) (width 0.2) (layer "B.Cu") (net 10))
 (segment (start 109.4622 60.602) (end 109.4622 57.3022) (width 0.2) (layer "B.Cu") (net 10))
 (segment (start 109.46 60.5998) (end 109.4622 60.602) (width 0.2) (layer "B.Cu") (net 10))
 (segment (start 114.5422 69.4854) (end 114.5422 72.5378) (width 0.2) (layer "B.Cu") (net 5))
 (segment (start 114.5422 72.5378) (end 114.54 72.54) (width 0.2) (layer "B.Cu") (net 5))
 (segment (start 113.65 65.57) (end 100.09 65.57) (width 0.2) (layer "F.Cu") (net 24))
 (via (at 100.09 65.57) (size 0.6) (drill 0.3) (layers "F.Cu" "B.Cu") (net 24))
 (via (at 113.65 65.57) (size 0.6) (drill 0.3) (layers "F.Cu" "B.Cu") (free yes) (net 24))
 (segment (start 114.5422 66.4622) (end 114.5422 67.4854) (width 0.2) (layer "B.Cu") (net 24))
 (segment (start 97.2702 65.57) (end 100.09 65.57) (width 0.2) (layer "B.Cu") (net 24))
 (segment (start 100.09 65.57) (end 100.08 65.57) (width 0.2) (layer "B.Cu") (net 24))
 (segment (start 113.65 65.57) (end 114.5422 66.4622) (width 0.2) (layer "B.Cu") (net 24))
 (segment (start 100.08 66.84) (end 100.75 66.17) (width 0.2) (layer "F.Cu") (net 29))
 (segment (start 100.75 66.17) (end 108.16 66.17) (width 0.2) (layer "F.Cu") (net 29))
 (via (at 100.08 66.84) (size 0.6) (drill 0.3) (layers "F.Cu" "B.Cu") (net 29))
 (via (at 108.16 66.17) (size 0.6) (drill 0.3) (layers "F.Cu" "B.Cu") (free yes) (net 29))
 (segment (start 108.16 66.17) (end 108.16 66.1832) (width 0.2) (layer "B.Cu") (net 29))
 (segment (start 97.2702 66.84) (end 100.08 66.84) (width 0.2) (layer "B.Cu") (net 29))
 (segment (start 108.16 66.1832) (end 109.4622 67.4854) (width 0.2) (layer "B.Cu") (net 29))
 (segment (start 109.4622 72.5378) (end 109.46 72.54) (width 0.2) (layer "B.Cu") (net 3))
 (segment (start 109.4622 69.4854) (end 109.4622 72.5378) (width 0.2) (layer "B.Cu") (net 3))
 (segment (start 126.51 67.71) (end 126.51 62.4) (width 0.2) (layer "F.Cu") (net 23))
 (segment (start 93.74 69.54) (end 124.68 69.54) (width 0.2) (layer "F.Cu") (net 23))
 (segment (start 124.68 69.54) (end 126.51 67.71) (width 0.2) (layer "F.Cu") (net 23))
 (via (at 126.51 62.4) (size 0.6) (drill 0.3) (layers "F.Cu" "B.Cu") (free yes) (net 23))
 (via (at 93.74 69.54) (size 0.6) (drill 0.3) (layers "F.Cu" "B.Cu") (free yes) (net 23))
 (segment (start 124.08 61.76) (end 125.87 61.76) (width 0.2) (layer "B.Cu") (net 23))
 (segment (start 125.87 61.76) (end 126.51 62.4) (width 0.2) (layer "B.Cu") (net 23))
 (segment (start 93.7002 69.54) (end 92.2702 68.11) (width 0.2) (layer "B.Cu") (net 23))
 (segment (start 93.74 69.54) (end 93.7002 69.54) (width 0.2) (layer "B.Cu") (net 23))
 (segment (start 125.079999 60.49) (end 124.08 60.49) (width 0.2) (layer "B.Cu") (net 6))
 (segment (start 119.68 59.259714) (end 120.389714 58.55) (width 0.2) (layer "B.Cu") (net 6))
 (segment (start 119.68 69.94) (end 119.68 59.259714) (width 0.2) (layer "B.Cu") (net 6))
 (segment (start 117.08 72.54) (end 119.68 69.94) (width 0.2) (layer "B.Cu") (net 6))
 (segment (start 125.38 58.879448) (end 125.38 60.189999) (width 0.2) (layer "B.Cu") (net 6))
 (segment (start 125.38 60.189999) (end 125.079999 60.49) (width 0.2) (layer "B.Cu") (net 6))
 (segment (start 125.050552 58.55) (end 125.38 58.879448) (width 0.2) (layer "B.Cu") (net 6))
 (segment (start 120.389714 58.55) (end 125.050552 58.55) (width 0.2) (layer "B.Cu") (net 6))
 (segment (start 129.08 60.49) (end 130.079999 60.49) (width 0.2) (layer "B.Cu") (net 9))
 (segment (start 130.38 58.79) (end 126.68 55.09) (width 0.2) (layer "B.Cu") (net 9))
 (segment (start 130.079999 60.49) (end 130.38 60.189999) (width 0.2) (layer "B.Cu") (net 9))
 (segment (start 126.68 55.09) (end 114.21 55.09) (width 0.2) (layer "B.Cu") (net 9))
 (segment (start 114.21 55.09) (end 112 57.3) (width 0.2) (layer "B.Cu") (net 9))
 (segment (start 130.38 60.189999) (end 130.38 58.79) (width 0.2) (layer "B.Cu") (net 9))
 (segment (start 129.08 61.76) (end 130.079999 61.76) (width 0.2) (layer "B.Cu") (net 12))
 (segment (start 107.19 54.49) (end 104.38 57.3) (width 0.2) (layer "B.Cu") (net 12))
 (segment (start 131.08 58.49) (end 127.08 54.49) (width 0.2) (layer "B.Cu") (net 12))
 (segment (start 127.08 54.49) (end 107.19 54.49) (width 0.2) (layer "B.Cu") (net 12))
 (segment (start 131.08 60.759999) (end 131.08 58.49) (width 0.2) (layer "B.Cu") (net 12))
 (segment (start 130.079999 61.76) (end 131.08 60.759999) (width 0.2) (layer "B.Cu") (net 12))
 (segment (start 116.35 55.49) (end 114.54 57.3) (width 0.2) (layer "B.Cu") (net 8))
 (segment (start 125.35 55.49) (end 116.35 55.49) (width 0.2) (layer "B.Cu") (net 8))
 (segment (start 129.08 59.22) (end 125.35 55.49) (width 0.2) (layer "B.Cu") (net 8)))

